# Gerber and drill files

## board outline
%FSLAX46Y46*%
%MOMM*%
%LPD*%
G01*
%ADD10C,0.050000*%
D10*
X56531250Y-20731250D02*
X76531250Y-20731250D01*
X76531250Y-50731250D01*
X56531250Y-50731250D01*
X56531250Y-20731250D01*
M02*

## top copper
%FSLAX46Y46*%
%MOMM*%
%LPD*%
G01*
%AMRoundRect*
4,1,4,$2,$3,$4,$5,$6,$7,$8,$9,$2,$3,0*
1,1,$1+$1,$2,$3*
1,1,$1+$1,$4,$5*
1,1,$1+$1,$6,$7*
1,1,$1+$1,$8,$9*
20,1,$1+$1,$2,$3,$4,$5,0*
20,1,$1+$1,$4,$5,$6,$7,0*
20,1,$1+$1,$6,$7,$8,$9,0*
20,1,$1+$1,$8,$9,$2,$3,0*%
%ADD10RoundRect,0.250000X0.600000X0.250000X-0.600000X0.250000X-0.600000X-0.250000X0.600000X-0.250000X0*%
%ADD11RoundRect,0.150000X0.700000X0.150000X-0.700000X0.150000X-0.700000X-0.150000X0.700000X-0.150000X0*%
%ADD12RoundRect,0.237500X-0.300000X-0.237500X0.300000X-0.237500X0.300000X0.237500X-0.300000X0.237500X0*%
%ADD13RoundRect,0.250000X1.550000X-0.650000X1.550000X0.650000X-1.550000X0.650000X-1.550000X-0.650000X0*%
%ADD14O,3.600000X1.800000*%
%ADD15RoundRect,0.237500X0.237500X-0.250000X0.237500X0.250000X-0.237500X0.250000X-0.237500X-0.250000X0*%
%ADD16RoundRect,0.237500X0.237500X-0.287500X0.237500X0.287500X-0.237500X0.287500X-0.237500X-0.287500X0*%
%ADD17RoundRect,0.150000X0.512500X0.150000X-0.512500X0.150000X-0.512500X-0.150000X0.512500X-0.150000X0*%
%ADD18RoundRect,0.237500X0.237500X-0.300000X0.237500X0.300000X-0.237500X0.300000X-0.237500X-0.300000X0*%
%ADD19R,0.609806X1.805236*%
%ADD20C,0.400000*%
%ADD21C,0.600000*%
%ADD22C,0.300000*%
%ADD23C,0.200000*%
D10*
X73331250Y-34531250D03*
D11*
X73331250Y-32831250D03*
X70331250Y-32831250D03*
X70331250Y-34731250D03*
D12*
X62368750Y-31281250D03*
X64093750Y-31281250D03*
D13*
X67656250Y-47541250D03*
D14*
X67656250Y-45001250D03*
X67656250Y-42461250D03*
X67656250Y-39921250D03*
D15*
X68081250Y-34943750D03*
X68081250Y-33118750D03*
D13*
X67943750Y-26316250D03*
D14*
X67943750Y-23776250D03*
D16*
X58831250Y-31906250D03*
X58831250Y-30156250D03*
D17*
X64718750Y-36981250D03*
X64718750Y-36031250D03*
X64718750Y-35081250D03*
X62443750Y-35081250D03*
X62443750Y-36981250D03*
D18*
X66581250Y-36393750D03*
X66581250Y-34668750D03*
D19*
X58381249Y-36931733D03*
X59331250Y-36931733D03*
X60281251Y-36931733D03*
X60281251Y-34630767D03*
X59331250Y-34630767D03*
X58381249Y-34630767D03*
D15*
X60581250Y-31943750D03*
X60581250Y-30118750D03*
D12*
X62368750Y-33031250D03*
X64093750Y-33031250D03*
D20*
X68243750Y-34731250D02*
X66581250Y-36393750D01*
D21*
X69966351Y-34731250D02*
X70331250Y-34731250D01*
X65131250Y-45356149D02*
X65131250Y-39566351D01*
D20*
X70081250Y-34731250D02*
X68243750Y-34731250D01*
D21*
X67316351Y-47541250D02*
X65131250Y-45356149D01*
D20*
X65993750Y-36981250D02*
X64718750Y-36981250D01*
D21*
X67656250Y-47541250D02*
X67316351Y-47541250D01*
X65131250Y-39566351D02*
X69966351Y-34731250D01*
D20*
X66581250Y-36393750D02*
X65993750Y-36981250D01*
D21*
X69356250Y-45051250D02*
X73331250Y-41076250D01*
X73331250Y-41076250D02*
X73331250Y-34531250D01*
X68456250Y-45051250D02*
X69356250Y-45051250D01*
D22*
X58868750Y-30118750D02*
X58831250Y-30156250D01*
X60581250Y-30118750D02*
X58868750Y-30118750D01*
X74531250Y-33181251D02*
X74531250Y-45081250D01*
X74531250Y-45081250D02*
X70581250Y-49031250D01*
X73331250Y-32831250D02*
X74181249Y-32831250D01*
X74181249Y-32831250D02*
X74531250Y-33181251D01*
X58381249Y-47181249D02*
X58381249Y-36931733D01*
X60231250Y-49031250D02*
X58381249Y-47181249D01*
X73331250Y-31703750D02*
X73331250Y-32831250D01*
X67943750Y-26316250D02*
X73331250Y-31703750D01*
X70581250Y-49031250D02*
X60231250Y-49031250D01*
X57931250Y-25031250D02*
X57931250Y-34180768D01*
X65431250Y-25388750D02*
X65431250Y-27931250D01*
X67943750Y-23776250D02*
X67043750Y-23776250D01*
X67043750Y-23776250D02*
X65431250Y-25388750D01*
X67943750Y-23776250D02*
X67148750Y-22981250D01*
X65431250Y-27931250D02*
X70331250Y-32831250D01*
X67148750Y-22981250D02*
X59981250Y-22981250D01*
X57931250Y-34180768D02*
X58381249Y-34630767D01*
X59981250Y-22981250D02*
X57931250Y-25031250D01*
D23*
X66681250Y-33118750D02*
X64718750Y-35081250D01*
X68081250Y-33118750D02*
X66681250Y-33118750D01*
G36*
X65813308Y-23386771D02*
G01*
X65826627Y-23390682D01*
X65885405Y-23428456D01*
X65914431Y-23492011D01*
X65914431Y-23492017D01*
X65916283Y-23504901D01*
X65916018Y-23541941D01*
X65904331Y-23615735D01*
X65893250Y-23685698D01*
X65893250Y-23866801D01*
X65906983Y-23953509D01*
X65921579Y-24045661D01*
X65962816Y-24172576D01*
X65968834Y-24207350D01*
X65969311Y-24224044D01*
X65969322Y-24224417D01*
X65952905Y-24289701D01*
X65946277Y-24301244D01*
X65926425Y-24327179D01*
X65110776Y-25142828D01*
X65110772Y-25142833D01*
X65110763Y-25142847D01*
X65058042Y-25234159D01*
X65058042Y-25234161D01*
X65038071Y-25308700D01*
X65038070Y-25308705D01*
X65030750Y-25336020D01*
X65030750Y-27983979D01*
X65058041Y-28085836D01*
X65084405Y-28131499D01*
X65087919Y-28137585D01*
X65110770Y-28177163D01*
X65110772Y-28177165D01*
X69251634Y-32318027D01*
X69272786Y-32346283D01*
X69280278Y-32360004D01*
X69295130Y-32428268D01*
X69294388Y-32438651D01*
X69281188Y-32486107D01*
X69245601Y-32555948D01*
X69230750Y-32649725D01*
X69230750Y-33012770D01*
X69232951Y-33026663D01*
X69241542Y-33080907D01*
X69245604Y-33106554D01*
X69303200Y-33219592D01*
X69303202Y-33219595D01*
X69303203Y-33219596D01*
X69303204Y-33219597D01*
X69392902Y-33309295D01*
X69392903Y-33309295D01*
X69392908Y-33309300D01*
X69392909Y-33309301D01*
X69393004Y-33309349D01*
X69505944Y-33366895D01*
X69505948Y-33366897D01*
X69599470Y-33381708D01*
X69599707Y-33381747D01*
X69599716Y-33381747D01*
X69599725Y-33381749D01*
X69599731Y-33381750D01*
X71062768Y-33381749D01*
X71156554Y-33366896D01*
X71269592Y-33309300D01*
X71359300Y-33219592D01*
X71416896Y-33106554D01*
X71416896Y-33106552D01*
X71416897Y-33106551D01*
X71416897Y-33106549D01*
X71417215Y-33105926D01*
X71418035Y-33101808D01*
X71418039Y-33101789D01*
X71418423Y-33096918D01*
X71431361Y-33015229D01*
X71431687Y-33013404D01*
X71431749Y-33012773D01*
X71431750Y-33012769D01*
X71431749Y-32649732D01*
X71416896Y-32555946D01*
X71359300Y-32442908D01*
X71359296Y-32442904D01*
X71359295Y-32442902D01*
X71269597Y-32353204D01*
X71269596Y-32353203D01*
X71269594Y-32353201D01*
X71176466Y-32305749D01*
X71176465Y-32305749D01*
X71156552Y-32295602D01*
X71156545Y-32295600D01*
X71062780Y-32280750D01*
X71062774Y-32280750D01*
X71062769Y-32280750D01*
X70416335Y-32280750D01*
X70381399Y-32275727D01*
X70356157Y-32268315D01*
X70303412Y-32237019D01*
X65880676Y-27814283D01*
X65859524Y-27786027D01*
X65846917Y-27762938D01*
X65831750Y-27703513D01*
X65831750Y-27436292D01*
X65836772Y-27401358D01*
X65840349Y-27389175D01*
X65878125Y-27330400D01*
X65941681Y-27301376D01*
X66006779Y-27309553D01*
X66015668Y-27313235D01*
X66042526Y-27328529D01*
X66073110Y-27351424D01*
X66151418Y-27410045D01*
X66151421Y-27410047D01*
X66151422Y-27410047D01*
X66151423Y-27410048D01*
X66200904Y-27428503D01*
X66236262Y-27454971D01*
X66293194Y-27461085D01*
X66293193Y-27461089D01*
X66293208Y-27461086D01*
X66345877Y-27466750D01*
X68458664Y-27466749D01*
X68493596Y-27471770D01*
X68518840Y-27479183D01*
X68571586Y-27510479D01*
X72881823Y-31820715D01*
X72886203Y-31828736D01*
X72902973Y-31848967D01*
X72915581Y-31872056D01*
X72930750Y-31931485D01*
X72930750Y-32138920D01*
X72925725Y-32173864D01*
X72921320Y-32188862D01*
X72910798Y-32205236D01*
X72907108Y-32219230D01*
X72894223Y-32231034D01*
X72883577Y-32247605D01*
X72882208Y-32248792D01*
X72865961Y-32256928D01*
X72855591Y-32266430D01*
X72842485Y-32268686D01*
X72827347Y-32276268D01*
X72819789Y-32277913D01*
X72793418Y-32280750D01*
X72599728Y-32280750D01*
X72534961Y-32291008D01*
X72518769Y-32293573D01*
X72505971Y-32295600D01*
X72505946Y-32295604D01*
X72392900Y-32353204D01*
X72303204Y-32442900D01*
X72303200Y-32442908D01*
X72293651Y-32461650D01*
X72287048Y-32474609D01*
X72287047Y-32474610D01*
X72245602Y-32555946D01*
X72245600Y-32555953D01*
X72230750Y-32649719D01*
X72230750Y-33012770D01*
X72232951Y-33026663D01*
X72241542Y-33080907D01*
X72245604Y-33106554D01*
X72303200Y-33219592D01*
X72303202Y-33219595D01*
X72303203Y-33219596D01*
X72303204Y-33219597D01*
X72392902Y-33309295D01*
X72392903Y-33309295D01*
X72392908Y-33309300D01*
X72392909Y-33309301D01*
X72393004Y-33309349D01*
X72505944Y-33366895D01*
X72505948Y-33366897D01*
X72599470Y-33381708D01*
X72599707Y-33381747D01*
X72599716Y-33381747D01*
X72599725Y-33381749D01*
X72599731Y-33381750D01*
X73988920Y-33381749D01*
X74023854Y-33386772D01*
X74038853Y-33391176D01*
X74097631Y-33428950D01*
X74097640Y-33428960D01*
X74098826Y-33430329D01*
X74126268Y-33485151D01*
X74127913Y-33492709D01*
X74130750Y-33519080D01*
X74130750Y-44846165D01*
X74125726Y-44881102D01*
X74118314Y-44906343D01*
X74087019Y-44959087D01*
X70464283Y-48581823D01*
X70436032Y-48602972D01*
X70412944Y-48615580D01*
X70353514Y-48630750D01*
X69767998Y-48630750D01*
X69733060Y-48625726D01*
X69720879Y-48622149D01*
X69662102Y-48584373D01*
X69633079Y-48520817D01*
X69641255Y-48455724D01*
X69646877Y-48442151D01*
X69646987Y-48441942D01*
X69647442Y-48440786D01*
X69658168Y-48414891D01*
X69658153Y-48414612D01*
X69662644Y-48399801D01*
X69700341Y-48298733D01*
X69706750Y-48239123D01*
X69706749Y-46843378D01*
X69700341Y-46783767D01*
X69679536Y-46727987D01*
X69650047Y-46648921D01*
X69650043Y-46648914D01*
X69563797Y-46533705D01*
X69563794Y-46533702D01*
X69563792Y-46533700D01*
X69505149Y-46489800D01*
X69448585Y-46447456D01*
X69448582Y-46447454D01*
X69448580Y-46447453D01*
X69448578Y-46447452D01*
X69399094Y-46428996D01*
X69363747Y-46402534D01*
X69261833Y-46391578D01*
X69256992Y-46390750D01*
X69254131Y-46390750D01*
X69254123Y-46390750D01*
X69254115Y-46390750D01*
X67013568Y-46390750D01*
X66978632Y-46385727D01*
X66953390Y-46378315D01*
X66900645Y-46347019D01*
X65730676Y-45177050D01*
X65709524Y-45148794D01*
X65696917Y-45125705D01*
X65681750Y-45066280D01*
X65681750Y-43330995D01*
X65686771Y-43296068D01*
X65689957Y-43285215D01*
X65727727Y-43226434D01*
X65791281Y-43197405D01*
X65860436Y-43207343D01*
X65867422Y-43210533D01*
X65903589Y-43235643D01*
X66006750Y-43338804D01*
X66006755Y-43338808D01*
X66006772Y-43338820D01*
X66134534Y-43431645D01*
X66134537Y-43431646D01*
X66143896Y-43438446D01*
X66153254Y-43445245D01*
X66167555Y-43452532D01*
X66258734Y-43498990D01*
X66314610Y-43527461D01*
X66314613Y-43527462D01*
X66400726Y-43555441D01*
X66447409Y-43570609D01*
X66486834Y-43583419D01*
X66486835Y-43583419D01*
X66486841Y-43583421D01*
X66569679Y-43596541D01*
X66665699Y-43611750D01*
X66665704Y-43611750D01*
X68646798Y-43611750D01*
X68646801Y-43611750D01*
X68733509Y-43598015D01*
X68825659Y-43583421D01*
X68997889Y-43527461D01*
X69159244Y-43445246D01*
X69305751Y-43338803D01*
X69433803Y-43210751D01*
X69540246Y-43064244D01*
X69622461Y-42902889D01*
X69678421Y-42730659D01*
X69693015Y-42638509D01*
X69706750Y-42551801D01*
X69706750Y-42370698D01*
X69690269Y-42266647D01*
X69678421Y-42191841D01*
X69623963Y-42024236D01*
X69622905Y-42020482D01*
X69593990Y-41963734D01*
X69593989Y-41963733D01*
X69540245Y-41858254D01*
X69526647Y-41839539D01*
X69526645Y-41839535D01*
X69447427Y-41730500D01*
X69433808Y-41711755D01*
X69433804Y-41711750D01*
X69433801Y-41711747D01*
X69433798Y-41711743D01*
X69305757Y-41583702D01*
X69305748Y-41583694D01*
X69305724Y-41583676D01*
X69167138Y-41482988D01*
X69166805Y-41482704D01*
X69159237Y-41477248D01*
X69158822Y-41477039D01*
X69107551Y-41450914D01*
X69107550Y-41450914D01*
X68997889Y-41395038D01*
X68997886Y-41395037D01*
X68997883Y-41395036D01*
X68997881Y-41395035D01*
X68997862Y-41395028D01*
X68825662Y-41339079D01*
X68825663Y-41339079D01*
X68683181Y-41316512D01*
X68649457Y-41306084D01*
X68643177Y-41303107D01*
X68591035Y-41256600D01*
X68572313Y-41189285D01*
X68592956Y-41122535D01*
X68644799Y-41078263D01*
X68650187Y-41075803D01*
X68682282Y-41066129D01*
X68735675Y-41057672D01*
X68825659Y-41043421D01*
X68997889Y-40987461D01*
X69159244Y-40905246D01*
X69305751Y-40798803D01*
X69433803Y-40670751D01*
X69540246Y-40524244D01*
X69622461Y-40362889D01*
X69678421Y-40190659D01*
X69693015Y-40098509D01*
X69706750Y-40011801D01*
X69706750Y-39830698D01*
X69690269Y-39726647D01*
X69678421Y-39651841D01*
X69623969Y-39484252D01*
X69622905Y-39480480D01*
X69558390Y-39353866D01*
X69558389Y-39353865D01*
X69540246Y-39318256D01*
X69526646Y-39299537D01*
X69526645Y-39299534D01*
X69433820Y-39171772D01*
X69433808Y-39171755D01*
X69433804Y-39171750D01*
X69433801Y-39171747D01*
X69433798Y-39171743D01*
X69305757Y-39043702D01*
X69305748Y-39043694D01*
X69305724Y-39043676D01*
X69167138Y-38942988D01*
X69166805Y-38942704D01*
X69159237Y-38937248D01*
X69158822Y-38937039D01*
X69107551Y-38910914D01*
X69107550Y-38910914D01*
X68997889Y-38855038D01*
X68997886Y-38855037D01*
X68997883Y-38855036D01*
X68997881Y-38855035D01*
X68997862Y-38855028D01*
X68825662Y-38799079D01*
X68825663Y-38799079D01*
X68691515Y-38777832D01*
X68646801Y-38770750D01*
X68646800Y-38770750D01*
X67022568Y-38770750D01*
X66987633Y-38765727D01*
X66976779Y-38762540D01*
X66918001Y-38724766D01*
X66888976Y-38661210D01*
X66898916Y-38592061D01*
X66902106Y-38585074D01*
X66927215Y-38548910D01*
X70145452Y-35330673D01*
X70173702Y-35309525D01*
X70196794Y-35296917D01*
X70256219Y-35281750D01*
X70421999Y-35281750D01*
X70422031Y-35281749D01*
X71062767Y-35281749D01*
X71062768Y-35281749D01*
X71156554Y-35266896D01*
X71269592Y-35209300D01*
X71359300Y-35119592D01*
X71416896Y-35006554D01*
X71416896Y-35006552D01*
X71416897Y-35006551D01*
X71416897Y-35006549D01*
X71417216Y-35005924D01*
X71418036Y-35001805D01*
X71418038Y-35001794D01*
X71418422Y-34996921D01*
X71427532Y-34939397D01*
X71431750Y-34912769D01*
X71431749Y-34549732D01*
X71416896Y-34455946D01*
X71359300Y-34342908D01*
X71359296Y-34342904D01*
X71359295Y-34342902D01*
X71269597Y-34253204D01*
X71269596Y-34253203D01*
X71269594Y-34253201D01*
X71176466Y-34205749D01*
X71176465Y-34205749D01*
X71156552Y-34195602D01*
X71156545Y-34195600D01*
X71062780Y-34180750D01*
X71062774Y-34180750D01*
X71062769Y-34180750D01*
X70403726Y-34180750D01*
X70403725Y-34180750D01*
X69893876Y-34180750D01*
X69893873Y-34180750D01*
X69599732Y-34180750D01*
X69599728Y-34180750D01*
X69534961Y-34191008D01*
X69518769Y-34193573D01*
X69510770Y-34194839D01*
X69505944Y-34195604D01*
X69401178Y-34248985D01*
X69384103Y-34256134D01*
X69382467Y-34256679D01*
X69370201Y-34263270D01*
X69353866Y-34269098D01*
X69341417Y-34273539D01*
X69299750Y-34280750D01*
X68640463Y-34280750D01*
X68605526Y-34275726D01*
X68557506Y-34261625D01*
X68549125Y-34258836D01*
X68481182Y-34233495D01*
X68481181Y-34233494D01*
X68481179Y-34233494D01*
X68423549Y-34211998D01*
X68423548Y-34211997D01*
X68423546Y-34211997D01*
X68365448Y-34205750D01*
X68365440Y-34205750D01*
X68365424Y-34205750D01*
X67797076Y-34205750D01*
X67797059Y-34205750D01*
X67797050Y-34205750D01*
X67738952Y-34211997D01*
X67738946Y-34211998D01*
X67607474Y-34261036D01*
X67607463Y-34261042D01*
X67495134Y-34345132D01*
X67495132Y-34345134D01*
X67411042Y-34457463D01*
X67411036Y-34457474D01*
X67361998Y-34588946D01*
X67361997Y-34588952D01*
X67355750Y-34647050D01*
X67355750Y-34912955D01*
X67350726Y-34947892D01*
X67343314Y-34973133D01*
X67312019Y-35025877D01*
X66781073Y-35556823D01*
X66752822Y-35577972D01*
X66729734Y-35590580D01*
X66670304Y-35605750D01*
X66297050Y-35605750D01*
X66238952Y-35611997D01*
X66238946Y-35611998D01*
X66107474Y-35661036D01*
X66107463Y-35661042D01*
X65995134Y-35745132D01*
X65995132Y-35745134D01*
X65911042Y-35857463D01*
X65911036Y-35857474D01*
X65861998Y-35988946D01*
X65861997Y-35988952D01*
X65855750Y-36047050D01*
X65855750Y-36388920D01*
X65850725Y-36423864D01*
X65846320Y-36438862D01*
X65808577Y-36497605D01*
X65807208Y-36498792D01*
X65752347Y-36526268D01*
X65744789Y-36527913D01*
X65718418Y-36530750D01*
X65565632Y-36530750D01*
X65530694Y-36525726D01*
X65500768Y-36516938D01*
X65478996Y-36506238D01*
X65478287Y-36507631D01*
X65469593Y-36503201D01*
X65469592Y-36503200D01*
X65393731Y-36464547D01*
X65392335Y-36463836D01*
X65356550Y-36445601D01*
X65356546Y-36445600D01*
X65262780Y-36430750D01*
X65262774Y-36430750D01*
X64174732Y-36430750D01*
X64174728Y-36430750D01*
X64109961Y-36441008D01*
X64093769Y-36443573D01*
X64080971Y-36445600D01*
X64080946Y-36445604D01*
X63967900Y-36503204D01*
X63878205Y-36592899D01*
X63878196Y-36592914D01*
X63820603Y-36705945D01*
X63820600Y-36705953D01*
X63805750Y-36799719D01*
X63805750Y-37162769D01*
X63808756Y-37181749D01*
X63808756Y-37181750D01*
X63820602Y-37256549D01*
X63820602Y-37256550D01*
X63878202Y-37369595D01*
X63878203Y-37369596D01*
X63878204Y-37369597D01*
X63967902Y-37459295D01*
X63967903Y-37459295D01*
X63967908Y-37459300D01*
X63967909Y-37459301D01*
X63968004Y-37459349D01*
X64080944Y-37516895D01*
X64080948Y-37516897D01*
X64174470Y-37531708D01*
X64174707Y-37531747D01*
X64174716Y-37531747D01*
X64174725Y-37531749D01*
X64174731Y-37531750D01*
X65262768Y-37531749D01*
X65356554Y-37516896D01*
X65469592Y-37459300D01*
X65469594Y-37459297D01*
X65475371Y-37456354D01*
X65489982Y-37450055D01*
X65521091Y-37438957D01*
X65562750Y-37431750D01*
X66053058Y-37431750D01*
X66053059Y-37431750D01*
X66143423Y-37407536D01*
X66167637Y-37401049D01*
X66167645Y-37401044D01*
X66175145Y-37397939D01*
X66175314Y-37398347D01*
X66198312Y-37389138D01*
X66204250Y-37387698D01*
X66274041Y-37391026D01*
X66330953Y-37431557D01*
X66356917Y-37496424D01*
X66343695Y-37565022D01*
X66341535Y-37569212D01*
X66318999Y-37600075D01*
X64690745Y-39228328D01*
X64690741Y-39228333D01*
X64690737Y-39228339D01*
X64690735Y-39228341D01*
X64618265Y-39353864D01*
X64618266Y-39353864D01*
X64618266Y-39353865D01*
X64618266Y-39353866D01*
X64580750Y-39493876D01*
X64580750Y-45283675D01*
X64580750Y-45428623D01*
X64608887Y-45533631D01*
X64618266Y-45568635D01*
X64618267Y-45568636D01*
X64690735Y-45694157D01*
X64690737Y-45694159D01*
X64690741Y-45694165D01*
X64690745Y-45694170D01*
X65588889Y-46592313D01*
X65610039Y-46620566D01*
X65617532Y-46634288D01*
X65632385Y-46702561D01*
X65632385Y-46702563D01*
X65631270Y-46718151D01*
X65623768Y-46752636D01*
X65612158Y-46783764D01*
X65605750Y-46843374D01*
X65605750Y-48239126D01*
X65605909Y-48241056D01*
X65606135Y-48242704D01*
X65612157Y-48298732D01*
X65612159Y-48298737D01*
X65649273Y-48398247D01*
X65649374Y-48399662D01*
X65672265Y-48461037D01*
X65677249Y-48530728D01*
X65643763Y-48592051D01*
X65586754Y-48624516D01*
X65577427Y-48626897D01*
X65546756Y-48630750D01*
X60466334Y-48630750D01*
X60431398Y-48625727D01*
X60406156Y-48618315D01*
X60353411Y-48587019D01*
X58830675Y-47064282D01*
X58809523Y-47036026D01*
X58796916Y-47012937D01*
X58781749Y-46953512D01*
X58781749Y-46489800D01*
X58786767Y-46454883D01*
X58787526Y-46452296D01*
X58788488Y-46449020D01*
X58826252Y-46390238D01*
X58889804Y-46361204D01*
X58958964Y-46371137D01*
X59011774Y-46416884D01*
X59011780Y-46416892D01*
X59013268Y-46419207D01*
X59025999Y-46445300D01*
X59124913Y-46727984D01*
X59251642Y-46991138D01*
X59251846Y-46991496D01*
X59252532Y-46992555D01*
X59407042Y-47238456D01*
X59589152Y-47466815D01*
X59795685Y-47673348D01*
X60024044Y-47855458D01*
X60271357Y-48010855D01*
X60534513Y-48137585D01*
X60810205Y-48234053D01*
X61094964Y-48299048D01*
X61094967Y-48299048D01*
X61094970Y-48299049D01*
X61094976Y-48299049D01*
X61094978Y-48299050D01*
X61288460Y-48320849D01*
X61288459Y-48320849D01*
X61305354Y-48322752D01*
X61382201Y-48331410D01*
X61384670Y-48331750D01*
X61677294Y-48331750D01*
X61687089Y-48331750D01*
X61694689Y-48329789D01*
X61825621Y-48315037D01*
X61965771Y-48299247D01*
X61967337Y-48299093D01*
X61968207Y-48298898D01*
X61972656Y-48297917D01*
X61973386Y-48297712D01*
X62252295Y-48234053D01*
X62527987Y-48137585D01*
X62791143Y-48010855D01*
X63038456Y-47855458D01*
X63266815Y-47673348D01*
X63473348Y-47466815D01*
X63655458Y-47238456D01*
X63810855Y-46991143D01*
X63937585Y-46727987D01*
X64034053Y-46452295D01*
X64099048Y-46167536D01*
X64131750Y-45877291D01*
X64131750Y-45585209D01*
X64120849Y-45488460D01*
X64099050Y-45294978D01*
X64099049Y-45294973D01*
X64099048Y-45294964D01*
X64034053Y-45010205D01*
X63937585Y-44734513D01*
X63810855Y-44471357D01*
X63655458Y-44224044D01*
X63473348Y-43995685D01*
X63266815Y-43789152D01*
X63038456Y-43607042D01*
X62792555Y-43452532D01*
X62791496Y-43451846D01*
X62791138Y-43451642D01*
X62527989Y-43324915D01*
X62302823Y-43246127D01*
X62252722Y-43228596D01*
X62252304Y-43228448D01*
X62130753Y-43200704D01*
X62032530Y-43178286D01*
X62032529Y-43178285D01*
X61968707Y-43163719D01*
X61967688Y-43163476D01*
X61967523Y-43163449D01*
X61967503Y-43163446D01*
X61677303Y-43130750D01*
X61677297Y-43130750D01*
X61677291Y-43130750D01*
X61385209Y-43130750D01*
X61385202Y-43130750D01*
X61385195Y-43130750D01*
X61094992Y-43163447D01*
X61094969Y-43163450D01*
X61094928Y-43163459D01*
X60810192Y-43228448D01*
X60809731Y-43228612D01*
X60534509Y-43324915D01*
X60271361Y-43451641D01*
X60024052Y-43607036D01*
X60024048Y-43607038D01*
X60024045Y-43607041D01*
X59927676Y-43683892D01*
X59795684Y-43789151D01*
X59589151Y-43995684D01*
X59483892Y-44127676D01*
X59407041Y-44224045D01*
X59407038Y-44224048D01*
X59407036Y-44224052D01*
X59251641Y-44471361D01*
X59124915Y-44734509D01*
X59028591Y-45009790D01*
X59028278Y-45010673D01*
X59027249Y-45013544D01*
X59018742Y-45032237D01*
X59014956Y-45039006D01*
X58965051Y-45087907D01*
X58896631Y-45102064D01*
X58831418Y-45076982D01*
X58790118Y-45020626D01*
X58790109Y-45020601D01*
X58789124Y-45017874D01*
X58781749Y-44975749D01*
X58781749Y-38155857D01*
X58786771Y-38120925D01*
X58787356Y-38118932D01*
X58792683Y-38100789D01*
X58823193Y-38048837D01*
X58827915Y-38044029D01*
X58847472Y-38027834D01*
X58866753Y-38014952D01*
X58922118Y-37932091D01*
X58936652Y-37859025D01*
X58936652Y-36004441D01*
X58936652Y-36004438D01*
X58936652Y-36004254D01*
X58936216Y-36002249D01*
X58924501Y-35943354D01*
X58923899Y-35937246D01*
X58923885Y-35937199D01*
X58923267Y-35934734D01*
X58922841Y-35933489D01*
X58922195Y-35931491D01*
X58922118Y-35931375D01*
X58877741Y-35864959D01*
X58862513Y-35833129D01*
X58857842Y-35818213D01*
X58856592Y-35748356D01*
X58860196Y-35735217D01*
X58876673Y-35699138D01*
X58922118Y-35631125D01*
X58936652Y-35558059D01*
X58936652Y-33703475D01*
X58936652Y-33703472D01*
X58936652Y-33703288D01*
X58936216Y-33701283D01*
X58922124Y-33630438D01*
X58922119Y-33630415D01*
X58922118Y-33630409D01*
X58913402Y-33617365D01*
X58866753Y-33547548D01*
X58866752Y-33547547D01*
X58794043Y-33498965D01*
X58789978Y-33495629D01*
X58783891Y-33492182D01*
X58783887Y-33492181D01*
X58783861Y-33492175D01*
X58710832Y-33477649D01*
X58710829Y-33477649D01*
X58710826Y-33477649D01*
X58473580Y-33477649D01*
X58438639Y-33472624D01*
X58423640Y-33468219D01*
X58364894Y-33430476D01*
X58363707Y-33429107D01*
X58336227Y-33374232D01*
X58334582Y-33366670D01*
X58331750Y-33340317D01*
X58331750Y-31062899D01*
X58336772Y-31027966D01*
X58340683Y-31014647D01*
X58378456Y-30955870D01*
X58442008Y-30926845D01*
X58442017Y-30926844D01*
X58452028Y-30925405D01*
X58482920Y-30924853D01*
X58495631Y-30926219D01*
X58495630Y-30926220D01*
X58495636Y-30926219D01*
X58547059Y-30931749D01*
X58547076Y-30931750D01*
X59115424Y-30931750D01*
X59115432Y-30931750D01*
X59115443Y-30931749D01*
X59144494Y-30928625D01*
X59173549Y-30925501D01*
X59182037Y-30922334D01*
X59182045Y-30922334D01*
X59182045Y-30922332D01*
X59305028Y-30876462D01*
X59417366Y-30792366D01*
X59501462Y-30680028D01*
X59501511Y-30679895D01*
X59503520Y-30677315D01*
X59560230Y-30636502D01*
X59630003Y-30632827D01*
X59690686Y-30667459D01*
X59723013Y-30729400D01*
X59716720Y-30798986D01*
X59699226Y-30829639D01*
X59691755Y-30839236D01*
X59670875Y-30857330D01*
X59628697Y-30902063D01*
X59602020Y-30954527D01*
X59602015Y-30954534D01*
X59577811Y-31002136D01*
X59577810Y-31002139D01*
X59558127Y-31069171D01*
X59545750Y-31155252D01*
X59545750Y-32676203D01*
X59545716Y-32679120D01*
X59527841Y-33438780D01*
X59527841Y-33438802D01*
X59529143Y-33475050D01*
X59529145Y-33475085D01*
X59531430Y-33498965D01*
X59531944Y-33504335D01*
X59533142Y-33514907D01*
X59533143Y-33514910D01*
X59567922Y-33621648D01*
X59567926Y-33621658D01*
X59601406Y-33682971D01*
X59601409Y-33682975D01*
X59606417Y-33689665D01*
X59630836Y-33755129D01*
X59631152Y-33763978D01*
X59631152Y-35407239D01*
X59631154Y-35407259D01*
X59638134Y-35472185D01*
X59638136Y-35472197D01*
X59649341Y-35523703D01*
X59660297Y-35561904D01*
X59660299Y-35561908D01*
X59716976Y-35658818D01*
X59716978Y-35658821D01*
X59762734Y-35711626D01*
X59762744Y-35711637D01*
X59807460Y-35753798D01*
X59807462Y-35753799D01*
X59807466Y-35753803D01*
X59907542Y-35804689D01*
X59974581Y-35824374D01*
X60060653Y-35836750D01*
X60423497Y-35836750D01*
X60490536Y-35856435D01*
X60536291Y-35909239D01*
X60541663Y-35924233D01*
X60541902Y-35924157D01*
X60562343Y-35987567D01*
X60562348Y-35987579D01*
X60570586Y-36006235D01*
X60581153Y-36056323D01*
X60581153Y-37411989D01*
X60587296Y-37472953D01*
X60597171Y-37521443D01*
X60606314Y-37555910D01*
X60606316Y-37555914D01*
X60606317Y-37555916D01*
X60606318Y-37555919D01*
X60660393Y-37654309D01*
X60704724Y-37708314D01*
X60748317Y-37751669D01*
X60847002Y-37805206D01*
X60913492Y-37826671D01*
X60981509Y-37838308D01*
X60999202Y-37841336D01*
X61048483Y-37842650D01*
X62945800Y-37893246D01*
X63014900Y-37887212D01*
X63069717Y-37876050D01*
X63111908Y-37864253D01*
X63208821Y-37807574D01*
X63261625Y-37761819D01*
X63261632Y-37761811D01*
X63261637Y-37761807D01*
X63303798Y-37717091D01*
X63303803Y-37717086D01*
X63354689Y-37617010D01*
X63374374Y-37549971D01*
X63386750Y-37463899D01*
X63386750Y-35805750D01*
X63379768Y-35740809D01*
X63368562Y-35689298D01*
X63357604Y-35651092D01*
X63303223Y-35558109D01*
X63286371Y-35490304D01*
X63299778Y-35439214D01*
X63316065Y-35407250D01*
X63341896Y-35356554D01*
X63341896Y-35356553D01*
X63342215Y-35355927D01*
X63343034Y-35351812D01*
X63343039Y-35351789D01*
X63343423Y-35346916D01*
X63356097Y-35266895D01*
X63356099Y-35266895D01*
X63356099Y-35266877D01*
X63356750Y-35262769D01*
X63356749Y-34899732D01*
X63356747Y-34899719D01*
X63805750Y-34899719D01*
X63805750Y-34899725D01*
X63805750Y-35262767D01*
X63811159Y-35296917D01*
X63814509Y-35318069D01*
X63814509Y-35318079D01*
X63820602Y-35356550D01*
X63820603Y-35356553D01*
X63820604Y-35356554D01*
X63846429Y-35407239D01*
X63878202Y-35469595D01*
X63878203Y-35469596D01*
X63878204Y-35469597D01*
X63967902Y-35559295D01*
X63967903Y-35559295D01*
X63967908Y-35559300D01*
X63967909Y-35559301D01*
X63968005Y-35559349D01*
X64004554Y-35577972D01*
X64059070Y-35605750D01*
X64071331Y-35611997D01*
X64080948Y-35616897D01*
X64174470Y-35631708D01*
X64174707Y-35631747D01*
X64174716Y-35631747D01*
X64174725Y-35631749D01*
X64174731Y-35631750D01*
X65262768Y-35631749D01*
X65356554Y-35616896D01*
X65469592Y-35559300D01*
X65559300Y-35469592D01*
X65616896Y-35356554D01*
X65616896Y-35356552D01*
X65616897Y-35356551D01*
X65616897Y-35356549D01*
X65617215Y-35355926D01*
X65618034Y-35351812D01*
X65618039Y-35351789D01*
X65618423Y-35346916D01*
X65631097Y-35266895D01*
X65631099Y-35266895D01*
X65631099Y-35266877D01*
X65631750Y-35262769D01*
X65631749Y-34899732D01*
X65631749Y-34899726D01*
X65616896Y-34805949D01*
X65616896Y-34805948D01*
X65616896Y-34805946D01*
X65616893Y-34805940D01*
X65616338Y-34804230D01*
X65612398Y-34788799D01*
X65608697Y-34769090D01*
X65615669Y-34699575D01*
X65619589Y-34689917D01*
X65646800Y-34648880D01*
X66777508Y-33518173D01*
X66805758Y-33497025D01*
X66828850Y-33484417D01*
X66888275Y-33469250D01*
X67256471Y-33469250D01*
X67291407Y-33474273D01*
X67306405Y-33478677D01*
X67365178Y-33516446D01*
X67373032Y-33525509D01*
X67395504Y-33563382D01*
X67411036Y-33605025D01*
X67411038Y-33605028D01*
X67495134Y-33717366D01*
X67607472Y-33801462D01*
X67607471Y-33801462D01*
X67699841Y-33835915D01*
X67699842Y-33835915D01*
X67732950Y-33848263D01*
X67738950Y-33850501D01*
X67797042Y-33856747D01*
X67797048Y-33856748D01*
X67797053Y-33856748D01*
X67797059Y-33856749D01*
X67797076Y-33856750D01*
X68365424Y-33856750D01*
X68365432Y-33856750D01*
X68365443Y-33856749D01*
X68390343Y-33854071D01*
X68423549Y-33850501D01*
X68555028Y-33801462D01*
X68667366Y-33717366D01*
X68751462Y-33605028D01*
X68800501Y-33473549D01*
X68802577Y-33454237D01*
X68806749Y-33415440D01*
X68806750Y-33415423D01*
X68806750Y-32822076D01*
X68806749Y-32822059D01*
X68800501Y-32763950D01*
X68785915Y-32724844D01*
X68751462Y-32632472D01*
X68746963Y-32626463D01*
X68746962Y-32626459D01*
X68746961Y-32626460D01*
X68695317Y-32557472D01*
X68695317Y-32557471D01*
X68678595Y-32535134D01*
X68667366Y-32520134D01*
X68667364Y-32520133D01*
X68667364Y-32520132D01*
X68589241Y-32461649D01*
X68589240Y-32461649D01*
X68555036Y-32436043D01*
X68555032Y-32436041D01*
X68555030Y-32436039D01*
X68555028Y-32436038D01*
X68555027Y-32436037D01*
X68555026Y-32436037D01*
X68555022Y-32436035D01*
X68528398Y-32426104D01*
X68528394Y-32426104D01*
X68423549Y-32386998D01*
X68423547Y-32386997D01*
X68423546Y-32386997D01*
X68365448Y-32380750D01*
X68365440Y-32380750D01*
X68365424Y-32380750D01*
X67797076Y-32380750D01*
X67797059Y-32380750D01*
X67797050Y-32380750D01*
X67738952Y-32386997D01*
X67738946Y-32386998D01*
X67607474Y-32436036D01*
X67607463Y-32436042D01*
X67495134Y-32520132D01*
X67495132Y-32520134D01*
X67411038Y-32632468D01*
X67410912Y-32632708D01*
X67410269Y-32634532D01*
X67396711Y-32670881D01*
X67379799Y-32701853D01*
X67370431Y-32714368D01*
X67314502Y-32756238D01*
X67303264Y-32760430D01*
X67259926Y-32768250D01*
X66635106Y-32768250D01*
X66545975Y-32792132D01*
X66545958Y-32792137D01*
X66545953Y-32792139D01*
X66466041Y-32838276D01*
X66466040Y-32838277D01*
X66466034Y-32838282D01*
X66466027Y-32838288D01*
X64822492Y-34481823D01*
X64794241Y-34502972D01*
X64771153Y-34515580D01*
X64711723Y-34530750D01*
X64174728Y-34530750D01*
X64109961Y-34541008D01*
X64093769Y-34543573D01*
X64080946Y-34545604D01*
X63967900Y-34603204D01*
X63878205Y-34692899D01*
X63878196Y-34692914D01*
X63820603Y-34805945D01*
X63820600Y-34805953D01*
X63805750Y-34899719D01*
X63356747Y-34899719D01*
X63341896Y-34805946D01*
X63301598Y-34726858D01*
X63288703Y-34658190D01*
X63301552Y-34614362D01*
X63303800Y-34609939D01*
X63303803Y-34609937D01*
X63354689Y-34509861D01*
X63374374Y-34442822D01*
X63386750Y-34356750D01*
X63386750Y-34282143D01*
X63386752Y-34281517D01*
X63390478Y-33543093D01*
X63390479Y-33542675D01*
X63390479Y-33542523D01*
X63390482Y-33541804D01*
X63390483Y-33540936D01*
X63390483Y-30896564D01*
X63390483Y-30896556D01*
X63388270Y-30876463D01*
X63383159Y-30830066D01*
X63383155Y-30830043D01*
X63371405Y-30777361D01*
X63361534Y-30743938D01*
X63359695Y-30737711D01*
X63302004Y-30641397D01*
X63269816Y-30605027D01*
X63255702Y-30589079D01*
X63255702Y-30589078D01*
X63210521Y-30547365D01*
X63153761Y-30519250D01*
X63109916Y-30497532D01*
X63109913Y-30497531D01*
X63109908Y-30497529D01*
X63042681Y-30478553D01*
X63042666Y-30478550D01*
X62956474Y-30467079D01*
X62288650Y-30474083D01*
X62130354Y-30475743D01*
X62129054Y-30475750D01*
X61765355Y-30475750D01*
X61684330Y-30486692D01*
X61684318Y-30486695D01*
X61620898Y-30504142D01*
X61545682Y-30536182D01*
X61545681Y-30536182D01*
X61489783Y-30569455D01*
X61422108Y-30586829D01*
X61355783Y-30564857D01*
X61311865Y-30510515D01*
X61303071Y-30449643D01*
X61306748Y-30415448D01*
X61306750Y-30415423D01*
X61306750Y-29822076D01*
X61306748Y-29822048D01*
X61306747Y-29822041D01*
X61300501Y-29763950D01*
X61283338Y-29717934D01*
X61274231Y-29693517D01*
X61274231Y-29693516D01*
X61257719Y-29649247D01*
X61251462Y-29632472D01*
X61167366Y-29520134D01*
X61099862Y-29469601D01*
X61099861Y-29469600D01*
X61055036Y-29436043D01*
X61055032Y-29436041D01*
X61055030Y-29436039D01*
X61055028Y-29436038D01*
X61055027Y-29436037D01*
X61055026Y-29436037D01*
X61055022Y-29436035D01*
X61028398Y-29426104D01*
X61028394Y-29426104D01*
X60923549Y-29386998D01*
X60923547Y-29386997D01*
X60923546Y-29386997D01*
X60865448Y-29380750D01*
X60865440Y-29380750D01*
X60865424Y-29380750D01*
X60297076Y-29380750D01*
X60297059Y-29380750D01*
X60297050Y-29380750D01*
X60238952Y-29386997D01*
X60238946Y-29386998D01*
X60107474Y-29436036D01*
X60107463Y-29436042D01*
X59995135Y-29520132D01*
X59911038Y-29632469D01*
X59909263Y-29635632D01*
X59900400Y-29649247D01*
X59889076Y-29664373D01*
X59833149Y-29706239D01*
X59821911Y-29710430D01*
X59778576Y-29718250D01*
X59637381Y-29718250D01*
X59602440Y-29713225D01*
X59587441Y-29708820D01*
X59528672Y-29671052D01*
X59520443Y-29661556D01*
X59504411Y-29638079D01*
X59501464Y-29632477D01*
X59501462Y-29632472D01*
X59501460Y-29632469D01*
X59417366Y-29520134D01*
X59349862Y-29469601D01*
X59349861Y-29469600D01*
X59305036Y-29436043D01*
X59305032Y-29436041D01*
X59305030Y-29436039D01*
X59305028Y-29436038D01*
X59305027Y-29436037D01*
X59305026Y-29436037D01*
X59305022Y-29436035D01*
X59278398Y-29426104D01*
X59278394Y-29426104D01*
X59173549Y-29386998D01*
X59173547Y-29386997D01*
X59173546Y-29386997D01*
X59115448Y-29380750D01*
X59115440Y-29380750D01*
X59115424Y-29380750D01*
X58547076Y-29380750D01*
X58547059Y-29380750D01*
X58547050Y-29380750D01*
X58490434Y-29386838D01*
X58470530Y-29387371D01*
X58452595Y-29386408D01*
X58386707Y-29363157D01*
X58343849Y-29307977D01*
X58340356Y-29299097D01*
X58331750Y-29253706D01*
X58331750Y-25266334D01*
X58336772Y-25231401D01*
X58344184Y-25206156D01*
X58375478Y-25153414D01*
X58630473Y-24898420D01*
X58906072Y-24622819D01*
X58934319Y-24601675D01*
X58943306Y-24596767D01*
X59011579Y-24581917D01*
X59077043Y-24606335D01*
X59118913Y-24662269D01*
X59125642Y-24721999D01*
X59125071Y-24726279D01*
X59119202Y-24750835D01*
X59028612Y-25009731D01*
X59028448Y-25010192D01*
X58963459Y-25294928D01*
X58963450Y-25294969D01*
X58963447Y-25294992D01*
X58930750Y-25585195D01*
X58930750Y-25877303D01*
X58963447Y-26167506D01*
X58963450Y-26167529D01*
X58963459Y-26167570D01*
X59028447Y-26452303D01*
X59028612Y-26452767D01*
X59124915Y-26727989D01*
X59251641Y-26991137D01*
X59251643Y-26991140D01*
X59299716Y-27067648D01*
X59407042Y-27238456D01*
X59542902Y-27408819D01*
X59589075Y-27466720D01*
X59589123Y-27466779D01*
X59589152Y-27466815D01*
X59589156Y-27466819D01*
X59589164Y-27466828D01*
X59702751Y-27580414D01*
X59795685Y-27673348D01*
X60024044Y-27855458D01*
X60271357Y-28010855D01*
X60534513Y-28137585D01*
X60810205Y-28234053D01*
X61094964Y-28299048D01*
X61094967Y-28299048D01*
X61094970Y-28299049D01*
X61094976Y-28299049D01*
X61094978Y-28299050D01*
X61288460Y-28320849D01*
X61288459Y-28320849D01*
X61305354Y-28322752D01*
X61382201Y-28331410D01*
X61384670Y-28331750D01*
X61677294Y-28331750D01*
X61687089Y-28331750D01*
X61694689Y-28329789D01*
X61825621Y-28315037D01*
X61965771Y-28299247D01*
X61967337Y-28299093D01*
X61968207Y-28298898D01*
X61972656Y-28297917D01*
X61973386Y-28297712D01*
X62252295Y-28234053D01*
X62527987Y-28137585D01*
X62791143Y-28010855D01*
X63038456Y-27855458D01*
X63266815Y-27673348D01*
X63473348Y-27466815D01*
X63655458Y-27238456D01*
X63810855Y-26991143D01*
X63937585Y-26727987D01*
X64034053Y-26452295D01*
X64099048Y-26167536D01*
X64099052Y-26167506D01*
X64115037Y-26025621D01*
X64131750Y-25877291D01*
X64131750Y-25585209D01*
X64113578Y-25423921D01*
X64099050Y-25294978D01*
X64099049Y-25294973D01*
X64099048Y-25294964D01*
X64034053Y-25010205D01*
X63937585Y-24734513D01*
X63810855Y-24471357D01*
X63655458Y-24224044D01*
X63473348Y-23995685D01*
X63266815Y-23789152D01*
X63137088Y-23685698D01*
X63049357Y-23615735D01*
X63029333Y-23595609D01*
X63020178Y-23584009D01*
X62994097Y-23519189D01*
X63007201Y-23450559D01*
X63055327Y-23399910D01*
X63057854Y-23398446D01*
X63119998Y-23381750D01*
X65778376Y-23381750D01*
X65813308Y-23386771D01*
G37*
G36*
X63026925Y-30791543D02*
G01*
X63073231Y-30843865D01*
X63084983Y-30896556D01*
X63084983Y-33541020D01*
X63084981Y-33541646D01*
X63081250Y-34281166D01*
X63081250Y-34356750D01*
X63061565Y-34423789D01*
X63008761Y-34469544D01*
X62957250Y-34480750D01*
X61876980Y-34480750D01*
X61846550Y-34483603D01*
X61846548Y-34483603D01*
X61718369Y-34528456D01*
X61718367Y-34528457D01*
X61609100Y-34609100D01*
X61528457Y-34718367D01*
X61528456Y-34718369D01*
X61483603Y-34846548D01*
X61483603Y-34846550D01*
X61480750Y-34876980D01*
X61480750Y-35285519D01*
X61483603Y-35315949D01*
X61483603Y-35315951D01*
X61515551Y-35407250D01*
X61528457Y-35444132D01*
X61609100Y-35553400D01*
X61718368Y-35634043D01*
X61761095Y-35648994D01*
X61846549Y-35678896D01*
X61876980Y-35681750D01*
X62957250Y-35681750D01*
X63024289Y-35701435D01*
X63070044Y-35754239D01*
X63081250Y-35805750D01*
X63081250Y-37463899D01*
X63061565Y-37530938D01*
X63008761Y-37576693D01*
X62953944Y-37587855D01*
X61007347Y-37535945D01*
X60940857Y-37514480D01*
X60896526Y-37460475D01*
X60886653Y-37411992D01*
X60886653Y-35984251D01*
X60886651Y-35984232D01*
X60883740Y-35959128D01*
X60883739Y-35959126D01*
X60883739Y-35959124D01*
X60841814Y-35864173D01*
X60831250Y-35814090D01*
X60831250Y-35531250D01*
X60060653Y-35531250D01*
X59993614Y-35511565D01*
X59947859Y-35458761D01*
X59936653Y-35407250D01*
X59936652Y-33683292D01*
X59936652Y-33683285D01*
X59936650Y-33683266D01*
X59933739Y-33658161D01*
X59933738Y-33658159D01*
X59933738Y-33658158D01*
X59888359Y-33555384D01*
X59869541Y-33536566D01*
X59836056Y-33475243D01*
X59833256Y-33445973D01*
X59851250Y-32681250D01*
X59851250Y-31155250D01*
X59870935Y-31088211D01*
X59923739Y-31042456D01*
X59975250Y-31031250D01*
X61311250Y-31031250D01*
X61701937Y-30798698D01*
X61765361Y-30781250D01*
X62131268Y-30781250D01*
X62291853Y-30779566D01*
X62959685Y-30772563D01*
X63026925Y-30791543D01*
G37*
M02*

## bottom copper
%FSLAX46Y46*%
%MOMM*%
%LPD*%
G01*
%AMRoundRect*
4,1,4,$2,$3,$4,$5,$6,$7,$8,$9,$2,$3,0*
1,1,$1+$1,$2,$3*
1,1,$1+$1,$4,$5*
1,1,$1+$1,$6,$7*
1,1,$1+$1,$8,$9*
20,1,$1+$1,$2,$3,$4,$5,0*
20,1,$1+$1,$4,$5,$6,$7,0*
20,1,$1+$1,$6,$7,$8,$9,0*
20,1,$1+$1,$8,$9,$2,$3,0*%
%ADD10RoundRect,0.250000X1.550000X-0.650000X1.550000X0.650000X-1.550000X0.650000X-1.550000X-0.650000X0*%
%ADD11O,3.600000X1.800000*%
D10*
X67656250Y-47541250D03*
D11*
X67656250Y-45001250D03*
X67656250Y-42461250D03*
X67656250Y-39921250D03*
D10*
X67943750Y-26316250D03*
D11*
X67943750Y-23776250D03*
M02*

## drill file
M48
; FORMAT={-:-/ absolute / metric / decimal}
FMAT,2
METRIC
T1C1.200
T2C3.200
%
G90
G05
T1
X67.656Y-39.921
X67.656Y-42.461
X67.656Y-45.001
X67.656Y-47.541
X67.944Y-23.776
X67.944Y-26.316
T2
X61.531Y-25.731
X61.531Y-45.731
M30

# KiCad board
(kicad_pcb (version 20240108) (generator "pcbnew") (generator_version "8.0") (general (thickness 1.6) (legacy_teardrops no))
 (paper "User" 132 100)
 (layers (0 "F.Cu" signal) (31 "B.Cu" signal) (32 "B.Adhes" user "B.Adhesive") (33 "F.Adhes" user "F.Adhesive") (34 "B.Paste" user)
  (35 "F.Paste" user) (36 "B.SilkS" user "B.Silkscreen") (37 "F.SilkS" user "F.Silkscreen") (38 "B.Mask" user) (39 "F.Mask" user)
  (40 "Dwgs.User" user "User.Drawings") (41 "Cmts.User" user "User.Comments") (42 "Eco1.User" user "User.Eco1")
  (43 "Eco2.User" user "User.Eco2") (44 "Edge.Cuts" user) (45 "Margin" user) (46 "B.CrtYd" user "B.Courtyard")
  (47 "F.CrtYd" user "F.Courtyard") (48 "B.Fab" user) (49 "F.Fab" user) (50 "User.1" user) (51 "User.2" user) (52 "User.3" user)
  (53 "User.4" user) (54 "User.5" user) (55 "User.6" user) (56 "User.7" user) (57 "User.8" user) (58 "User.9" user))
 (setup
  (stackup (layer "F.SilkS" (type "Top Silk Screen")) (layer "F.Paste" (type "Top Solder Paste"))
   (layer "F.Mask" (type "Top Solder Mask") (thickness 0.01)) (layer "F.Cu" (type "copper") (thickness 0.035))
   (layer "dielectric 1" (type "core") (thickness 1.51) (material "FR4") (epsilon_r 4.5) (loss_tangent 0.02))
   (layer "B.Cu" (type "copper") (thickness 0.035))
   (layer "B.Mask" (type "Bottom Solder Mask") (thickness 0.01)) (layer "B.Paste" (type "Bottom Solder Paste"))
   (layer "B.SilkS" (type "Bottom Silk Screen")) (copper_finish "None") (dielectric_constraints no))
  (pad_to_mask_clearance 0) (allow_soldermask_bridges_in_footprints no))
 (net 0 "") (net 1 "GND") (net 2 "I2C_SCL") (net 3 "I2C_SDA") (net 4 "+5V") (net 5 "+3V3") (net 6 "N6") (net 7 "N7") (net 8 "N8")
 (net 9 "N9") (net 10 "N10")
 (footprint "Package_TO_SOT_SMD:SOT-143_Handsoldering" (layer "F.Cu") (at 71.83125 33.78125 180)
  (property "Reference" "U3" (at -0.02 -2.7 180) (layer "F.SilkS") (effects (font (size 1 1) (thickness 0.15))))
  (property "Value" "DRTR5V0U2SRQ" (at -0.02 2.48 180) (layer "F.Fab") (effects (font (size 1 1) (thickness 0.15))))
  (pad "1" smd roundrect (at -1.5 -0.75 180) (size 1.7 1) (layers "F.Cu" "F.Paste" "F.Mask") (roundrect_rratio 0.25) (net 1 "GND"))
  (pad "2" smd roundrect (at -1.5 0.95 180) (size 1.7 0.6) (layers "F.Cu" "F.Paste" "F.Mask") (roundrect_rratio 0.25) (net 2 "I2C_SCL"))
  (pad "3" smd roundrect (at 1.5 0.95 180) (size 1.7 0.6) (layers "F.Cu" "F.Paste" "F.Mask") (roundrect_rratio 0.25) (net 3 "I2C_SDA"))
  (pad "4" smd roundrect (at 1.5 -0.95 180) (size 1.7 0.6) (layers "F.Cu" "F.Paste" "F.Mask") (roundrect_rratio 0.25) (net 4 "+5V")))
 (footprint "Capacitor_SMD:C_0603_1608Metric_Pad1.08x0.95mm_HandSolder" (layer "F.Cu") (at 63.23125 31.28125)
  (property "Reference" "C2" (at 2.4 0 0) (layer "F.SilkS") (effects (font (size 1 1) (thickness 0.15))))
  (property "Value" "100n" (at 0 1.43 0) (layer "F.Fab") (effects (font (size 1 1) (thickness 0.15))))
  (pad "1" smd roundrect (at -0.8625 0) (size 1.075 0.95) (layers "F.Cu" "F.Paste" "F.Mask") (roundrect_rratio 0.25) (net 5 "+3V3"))
  (pad "2" smd roundrect (at 0.8625 0) (size 1.075 0.95) (layers "F.Cu" "F.Paste" "F.Mask") (roundrect_rratio 0.25) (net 1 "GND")))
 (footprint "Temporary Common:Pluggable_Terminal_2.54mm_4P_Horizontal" (layer "F.Cu") (at 64.20625 43.51125 90)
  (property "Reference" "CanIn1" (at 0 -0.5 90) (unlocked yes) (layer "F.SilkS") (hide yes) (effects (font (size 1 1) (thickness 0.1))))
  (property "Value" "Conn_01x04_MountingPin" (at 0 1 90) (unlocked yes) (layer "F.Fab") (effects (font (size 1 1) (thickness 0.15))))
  (pad "1" thru_hole roundrect (at -4.03 3.45 90) (size 1.8 3.6) (drill 1.2) (layers "*.Cu" "*.Mask") (remove_unused_layers no)
   (roundrect_rratio 0.138889) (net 4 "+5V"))
  (pad "2" thru_hole oval (at -1.49 3.45 90) (size 1.8 3.6) (drill 1.2) (layers "*.Cu" "*.Mask") (remove_unused_layers no) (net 1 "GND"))
  (pad "3" thru_hole oval (at 1.05 3.45 90) (size 1.8 3.6) (drill 1.2) (layers "*.Cu" "*.Mask") (remove_unused_layers no) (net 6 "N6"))
  (pad "4" thru_hole oval (at 3.59 3.45 90) (size 1.8 3.6) (drill 1.2) (layers "*.Cu" "*.Mask") (remove_unused_layers no) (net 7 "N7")))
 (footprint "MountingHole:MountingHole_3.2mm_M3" (layer "F.Cu") (at 61.53125 25.73125)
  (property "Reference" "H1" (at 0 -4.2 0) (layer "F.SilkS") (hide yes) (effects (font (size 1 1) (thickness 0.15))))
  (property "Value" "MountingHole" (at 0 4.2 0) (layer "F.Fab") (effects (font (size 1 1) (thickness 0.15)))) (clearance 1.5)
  (pad "" np_thru_hole circle (at 0 0) (size 3.2 3.2) (drill 3.2) (layers "F&B.Cu" "*.Mask") (clearance 1)))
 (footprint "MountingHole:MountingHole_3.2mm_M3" (layer "F.Cu") (at 61.53125 45.73125)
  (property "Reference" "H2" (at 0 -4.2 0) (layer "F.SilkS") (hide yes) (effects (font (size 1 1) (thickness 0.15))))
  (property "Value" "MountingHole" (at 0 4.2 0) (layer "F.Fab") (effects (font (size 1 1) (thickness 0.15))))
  (pad "" np_thru_hole circle (at 0 0) (size 3.2 3.2) (drill 3.2) (layers "F&B.Cu" "*.Mask") (clearance 1)))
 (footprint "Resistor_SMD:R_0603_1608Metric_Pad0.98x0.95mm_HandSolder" (layer "F.Cu") (at 68.08125 34.03125 90)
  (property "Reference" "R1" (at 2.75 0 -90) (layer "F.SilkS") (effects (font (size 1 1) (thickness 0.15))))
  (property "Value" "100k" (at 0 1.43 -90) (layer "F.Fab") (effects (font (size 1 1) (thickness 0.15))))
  (pad "1" smd roundrect (at -0.9125 0 90) (size 0.975 0.95) (layers "F.Cu" "F.Paste" "F.Mask") (roundrect_rratio 0.25) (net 4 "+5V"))
  (pad "2" smd roundrect (at 0.9125 0 90) (size 0.975 0.95) (layers "F.Cu" "F.Paste" "F.Mask") (roundrect_rratio 0.25) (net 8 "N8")))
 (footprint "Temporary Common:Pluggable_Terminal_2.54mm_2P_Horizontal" (layer "F.Cu") (at 62.64375 24.48625 90)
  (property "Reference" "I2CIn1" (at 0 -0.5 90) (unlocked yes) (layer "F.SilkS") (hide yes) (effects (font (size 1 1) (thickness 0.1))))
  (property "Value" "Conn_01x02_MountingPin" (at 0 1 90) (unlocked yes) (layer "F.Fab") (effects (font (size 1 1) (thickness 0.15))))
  (pad "1" thru_hole roundrect (at -1.83 5.3 90) (size 1.8 3.6) (drill 1.2) (layers "*.Cu" "*.Mask") (remove_unused_layers no)
   (roundrect_rratio 0.138889) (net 2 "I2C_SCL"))
  (pad "2" thru_hole oval (at 0.71 5.3 90) (size 1.8 3.6) (drill 1.2) (layers "*.Cu" "*.Mask") (remove_unused_layers no) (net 3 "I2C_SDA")))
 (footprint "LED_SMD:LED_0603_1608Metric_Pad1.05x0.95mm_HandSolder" (layer "F.Cu") (at 58.83125 31.03125 90)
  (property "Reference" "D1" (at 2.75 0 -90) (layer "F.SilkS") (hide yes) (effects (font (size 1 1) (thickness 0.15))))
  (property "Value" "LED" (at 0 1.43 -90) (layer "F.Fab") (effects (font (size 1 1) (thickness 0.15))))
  (pad "1" smd roundrect (at -0.875 0 90) (size 1.05 0.95) (layers "F.Cu" "F.Paste" "F.Mask") (roundrect_rratio 0.25) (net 1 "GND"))
  (pad "2" smd roundrect (at 0.875 0 90) (size 1.05 0.95) (layers "F.Cu" "F.Paste" "F.Mask") (roundrect_rratio 0.25) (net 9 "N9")))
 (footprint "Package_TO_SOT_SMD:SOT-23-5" (layer "F.Cu") (at 63.58125 36.03125 180)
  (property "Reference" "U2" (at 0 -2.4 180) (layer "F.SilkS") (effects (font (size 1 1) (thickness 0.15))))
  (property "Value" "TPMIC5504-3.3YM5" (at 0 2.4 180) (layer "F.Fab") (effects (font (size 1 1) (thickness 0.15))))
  (pad "1" smd roundrect (at -1.1375 -0.95 180) (size 1.325 0.6) (layers "F.Cu" "F.Paste" "F.Mask") (roundrect_rratio 0.25) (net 4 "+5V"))
  (pad "2" smd roundrect (at -1.1375 0 180) (size 1.325 0.6) (layers "F.Cu" "F.Paste" "F.Mask") (roundrect_rratio 0.25) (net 1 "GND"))
  (pad "3" smd roundrect (at -1.1375 0.95 180) (size 1.325 0.6) (layers "F.Cu" "F.Paste" "F.Mask") (roundrect_rratio 0.25) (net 8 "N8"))
  (pad "4" smd roundrect (at 1.1375 0.95 180) (size 1.325 0.6) (layers "F.Cu" "F.Paste" "F.Mask") (roundrect_rratio 0.25) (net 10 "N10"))
  (pad "5" smd roundrect (at 1.1375 -0.95 180) (size 1.325 0.6) (layers "F.Cu" "F.Paste" "F.Mask") (roundrect_rratio 0.25) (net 5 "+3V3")))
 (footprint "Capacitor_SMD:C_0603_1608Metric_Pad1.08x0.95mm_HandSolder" (layer "F.Cu") (at 66.58125 35.53125 90)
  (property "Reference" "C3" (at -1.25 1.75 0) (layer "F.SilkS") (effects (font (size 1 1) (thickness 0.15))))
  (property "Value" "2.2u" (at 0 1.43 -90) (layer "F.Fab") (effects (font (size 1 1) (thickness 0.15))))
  (pad "1" smd roundrect (at -0.8625 0 90) (size 1.075 0.95) (layers "F.Cu" "F.Paste" "F.Mask") (roundrect_rratio 0.25) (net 4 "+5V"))
  (pad "2" smd roundrect (at 0.8625 0 90) (size 1.075 0.95) (layers "F.Cu" "F.Paste" "F.Mask") (roundrect_rratio 0.25) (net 1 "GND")))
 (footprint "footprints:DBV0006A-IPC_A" (layer "F.Cu") (at 59.33125 35.78125 90)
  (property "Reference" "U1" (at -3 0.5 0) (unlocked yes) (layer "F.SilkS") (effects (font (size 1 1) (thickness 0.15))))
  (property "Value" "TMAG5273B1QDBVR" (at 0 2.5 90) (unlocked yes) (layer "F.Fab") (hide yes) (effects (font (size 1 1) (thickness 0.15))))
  (pad "1" smd rect (at -1.150483 -0.950001 90) (size 1.805236 0.609806) (layers "F.Cu" "F.Paste" "F.Mask") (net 2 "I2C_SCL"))
  (pad "2" smd rect (at -1.150483 0 90) (size 1.805236 0.609806) (layers "F.Cu" "F.Paste" "F.Mask") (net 1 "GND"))
  (pad "3" smd rect (at -1.150483 0.950001 90) (size 1.805236 0.609806) (layers "F.Cu" "F.Paste" "F.Mask") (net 1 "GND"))
  (pad "4" smd rect (at 1.150483 0.950001 90) (size 1.805236 0.609806) (layers "F.Cu" "F.Paste" "F.Mask") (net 5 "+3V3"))
  (pad "5" smd rect (at 1.150483 0 90) (size 1.805236 0.609806) (layers "F.Cu" "F.Paste" "F.Mask") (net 1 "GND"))
  (pad "6" smd rect (at 1.150483 -0.950001 90) (size 1.805236 0.609806) (layers "F.Cu" "F.Paste" "F.Mask") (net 3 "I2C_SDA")))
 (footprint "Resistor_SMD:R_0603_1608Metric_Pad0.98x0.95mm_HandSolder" (layer "F.Cu") (at 60.58125 31.03125 90)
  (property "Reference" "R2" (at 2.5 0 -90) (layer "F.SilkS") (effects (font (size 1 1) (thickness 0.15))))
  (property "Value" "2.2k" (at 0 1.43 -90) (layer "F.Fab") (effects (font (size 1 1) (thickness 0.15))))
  (pad "1" smd roundrect (at -0.9125 0 90) (size 0.975 0.95) (layers "F.Cu" "F.Paste" "F.Mask") (roundrect_rratio 0.25) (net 5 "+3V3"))
  (pad "2" smd roundrect (at 0.9125 0 90) (size 0.975 0.95) (layers "F.Cu" "F.Paste" "F.Mask") (roundrect_rratio 0.25) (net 9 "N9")))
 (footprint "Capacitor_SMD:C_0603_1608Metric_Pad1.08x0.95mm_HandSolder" (layer "F.Cu") (at 63.23125 33.03125)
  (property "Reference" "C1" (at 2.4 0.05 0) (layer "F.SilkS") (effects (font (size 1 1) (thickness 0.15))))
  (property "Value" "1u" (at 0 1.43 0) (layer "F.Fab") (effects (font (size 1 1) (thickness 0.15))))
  (pad "1" smd roundrect (at -0.8625 0) (size 1.075 0.95) (layers "F.Cu" "F.Paste" "F.Mask") (roundrect_rratio 0.25) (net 5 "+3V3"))
  (pad "2" smd roundrect (at 0.8625 0) (size 1.075 0.95) (layers "F.Cu" "F.Paste" "F.Mask") (roundrect_rratio 0.25) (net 1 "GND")))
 (gr_rect (start 56.53125 20.73125) (end 76.53125 50.73125) (stroke (width 0.05) (type default)) (fill none) (layer "Edge.Cuts"))
 (segment (start 68.24375 34.73125) (end 66.58125 36.39375) (width 0.4) (layer "F.Cu") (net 4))
 (segment (start 69.966351 34.73125) (end 70.33125 34.73125) (width 0.6) (layer "F.Cu") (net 4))
 (segment (start 65.13125 45.356149) (end 65.13125 39.566351) (width 0.6) (layer "F.Cu") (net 4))
 (segment (start 70.08125 34.73125) (end 68.24375 34.73125) (width 0.4) (layer "F.Cu") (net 4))
 (segment (start 67.316351 47.54125) (end 65.13125 45.356149) (width 0.6) (layer "F.Cu") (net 4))
 (segment (start 65.99375 36.98125) (end 64.71875 36.98125) (width 0.4) (layer "F.Cu") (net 4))
 (segment (start 67.65625 47.54125) (end 67.316351 47.54125) (width 0.6) (layer "F.Cu") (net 4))
 (segment (start 65.13125 39.566351) (end 69.966351 34.73125) (width 0.6) (layer "F.Cu") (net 4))
 (segment (start 66.58125 36.39375) (end 65.99375 36.98125) (width 0.4) (layer "F.Cu") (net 4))
 (segment (start 69.35625 45.05125) (end 73.33125 41.07625) (width 0.6) (layer "F.Cu") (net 1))
 (segment (start 73.33125 41.07625) (end 73.33125 34.53125) (width 0.6) (layer "F.Cu") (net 1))
 (segment (start 68.45625 45.05125) (end 69.35625 45.05125) (width 0.6) (layer "F.Cu") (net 1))
 (segment (start 58.86875 30.11875) (end 58.83125 30.15625) (width 0.3) (layer "F.Cu") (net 9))
 (segment (start 60.58125 30.11875) (end 58.86875 30.11875) (width 0.3) (layer "F.Cu") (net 9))
 (segment (start 74.53125 33.181251) (end 74.53125 45.08125) (width 0.3) (layer "F.Cu") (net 2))
 (segment (start 74.53125 45.08125) (end 70.58125 49.03125) (width 0.3) (layer "F.Cu") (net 2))
 (segment (start 73.33125 32.83125) (end 74.181249 32.83125) (width 0.3) (layer "F.Cu") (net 2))
 (segment (start 74.181249 32.83125) (end 74.53125 33.181251) (width 0.3) (layer "F.Cu") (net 2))
 (segment (start 58.381249 47.181249) (end 58.381249 36.931733) (width 0.3) (layer "F.Cu") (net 2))
 (segment (start 60.23125 49.03125) (end 58.381249 47.181249) (width 0.3) (layer "F.Cu") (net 2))
 (segment (start 73.33125 31.70375) (end 73.33125 32.83125) (width 0.3) (layer "F.Cu") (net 2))
 (segment (start 67.94375 26.31625) (end 73.33125 31.70375) (width 0.3) (layer "F.Cu") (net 2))
 (segment (start 70.58125 49.03125) (end 60.23125 49.03125) (width 0.3) (layer "F.Cu") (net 2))
 (segment (start 57.93125 25.03125) (end 57.93125 34.180768) (width 0.3) (layer "F.Cu") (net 3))
 (segment (start 65.43125 25.38875) (end 65.43125 27.93125) (width 0.3) (layer "F.Cu") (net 3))
 (segment (start 67.94375 23.77625) (end 67.04375 23.77625) (width 0.3) (layer "F.Cu") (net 3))
 (segment (start 67.04375 23.77625) (end 65.43125 25.38875) (width 0.3) (layer "F.Cu") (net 3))
 (segment (start 67.94375 23.77625) (end 67.14875 22.98125) (width 0.3) (layer "F.Cu") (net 3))
 (segment (start 65.43125 27.93125) (end 70.33125 32.83125) (width 0.3) (layer "F.Cu") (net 3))
 (segment (start 67.14875 22.98125) (end 59.98125 22.98125) (width 0.3) (layer "F.Cu") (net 3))
 (segment (start 57.93125 34.180768) (end 58.381249 34.630767) (width 0.3) (layer "F.Cu") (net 3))
 (segment (start 59.98125 22.98125) (end 57.93125 25.03125) (width 0.3) (layer "F.Cu") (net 3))
 (segment (start 66.68125 33.11875) (end 64.71875 35.08125) (width 0.2) (layer "F.Cu") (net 8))
 (segment (start 68.08125 33.11875) (end 66.68125 33.11875) (width 0.2) (layer "F.Cu") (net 8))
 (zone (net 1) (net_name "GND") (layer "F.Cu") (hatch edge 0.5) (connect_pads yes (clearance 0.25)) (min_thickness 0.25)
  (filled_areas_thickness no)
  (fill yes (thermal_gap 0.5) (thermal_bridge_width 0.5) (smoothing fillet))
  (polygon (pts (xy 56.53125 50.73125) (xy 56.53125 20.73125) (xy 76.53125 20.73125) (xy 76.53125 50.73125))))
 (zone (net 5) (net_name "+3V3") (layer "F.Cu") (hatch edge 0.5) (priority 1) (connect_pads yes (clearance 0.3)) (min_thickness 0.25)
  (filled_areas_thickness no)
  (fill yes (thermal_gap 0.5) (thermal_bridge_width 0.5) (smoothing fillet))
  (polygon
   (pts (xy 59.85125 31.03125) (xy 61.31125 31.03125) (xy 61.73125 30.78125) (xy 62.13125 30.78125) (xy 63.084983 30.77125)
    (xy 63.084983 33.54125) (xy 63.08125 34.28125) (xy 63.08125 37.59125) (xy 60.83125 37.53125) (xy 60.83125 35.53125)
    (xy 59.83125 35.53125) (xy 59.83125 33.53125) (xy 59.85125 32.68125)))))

